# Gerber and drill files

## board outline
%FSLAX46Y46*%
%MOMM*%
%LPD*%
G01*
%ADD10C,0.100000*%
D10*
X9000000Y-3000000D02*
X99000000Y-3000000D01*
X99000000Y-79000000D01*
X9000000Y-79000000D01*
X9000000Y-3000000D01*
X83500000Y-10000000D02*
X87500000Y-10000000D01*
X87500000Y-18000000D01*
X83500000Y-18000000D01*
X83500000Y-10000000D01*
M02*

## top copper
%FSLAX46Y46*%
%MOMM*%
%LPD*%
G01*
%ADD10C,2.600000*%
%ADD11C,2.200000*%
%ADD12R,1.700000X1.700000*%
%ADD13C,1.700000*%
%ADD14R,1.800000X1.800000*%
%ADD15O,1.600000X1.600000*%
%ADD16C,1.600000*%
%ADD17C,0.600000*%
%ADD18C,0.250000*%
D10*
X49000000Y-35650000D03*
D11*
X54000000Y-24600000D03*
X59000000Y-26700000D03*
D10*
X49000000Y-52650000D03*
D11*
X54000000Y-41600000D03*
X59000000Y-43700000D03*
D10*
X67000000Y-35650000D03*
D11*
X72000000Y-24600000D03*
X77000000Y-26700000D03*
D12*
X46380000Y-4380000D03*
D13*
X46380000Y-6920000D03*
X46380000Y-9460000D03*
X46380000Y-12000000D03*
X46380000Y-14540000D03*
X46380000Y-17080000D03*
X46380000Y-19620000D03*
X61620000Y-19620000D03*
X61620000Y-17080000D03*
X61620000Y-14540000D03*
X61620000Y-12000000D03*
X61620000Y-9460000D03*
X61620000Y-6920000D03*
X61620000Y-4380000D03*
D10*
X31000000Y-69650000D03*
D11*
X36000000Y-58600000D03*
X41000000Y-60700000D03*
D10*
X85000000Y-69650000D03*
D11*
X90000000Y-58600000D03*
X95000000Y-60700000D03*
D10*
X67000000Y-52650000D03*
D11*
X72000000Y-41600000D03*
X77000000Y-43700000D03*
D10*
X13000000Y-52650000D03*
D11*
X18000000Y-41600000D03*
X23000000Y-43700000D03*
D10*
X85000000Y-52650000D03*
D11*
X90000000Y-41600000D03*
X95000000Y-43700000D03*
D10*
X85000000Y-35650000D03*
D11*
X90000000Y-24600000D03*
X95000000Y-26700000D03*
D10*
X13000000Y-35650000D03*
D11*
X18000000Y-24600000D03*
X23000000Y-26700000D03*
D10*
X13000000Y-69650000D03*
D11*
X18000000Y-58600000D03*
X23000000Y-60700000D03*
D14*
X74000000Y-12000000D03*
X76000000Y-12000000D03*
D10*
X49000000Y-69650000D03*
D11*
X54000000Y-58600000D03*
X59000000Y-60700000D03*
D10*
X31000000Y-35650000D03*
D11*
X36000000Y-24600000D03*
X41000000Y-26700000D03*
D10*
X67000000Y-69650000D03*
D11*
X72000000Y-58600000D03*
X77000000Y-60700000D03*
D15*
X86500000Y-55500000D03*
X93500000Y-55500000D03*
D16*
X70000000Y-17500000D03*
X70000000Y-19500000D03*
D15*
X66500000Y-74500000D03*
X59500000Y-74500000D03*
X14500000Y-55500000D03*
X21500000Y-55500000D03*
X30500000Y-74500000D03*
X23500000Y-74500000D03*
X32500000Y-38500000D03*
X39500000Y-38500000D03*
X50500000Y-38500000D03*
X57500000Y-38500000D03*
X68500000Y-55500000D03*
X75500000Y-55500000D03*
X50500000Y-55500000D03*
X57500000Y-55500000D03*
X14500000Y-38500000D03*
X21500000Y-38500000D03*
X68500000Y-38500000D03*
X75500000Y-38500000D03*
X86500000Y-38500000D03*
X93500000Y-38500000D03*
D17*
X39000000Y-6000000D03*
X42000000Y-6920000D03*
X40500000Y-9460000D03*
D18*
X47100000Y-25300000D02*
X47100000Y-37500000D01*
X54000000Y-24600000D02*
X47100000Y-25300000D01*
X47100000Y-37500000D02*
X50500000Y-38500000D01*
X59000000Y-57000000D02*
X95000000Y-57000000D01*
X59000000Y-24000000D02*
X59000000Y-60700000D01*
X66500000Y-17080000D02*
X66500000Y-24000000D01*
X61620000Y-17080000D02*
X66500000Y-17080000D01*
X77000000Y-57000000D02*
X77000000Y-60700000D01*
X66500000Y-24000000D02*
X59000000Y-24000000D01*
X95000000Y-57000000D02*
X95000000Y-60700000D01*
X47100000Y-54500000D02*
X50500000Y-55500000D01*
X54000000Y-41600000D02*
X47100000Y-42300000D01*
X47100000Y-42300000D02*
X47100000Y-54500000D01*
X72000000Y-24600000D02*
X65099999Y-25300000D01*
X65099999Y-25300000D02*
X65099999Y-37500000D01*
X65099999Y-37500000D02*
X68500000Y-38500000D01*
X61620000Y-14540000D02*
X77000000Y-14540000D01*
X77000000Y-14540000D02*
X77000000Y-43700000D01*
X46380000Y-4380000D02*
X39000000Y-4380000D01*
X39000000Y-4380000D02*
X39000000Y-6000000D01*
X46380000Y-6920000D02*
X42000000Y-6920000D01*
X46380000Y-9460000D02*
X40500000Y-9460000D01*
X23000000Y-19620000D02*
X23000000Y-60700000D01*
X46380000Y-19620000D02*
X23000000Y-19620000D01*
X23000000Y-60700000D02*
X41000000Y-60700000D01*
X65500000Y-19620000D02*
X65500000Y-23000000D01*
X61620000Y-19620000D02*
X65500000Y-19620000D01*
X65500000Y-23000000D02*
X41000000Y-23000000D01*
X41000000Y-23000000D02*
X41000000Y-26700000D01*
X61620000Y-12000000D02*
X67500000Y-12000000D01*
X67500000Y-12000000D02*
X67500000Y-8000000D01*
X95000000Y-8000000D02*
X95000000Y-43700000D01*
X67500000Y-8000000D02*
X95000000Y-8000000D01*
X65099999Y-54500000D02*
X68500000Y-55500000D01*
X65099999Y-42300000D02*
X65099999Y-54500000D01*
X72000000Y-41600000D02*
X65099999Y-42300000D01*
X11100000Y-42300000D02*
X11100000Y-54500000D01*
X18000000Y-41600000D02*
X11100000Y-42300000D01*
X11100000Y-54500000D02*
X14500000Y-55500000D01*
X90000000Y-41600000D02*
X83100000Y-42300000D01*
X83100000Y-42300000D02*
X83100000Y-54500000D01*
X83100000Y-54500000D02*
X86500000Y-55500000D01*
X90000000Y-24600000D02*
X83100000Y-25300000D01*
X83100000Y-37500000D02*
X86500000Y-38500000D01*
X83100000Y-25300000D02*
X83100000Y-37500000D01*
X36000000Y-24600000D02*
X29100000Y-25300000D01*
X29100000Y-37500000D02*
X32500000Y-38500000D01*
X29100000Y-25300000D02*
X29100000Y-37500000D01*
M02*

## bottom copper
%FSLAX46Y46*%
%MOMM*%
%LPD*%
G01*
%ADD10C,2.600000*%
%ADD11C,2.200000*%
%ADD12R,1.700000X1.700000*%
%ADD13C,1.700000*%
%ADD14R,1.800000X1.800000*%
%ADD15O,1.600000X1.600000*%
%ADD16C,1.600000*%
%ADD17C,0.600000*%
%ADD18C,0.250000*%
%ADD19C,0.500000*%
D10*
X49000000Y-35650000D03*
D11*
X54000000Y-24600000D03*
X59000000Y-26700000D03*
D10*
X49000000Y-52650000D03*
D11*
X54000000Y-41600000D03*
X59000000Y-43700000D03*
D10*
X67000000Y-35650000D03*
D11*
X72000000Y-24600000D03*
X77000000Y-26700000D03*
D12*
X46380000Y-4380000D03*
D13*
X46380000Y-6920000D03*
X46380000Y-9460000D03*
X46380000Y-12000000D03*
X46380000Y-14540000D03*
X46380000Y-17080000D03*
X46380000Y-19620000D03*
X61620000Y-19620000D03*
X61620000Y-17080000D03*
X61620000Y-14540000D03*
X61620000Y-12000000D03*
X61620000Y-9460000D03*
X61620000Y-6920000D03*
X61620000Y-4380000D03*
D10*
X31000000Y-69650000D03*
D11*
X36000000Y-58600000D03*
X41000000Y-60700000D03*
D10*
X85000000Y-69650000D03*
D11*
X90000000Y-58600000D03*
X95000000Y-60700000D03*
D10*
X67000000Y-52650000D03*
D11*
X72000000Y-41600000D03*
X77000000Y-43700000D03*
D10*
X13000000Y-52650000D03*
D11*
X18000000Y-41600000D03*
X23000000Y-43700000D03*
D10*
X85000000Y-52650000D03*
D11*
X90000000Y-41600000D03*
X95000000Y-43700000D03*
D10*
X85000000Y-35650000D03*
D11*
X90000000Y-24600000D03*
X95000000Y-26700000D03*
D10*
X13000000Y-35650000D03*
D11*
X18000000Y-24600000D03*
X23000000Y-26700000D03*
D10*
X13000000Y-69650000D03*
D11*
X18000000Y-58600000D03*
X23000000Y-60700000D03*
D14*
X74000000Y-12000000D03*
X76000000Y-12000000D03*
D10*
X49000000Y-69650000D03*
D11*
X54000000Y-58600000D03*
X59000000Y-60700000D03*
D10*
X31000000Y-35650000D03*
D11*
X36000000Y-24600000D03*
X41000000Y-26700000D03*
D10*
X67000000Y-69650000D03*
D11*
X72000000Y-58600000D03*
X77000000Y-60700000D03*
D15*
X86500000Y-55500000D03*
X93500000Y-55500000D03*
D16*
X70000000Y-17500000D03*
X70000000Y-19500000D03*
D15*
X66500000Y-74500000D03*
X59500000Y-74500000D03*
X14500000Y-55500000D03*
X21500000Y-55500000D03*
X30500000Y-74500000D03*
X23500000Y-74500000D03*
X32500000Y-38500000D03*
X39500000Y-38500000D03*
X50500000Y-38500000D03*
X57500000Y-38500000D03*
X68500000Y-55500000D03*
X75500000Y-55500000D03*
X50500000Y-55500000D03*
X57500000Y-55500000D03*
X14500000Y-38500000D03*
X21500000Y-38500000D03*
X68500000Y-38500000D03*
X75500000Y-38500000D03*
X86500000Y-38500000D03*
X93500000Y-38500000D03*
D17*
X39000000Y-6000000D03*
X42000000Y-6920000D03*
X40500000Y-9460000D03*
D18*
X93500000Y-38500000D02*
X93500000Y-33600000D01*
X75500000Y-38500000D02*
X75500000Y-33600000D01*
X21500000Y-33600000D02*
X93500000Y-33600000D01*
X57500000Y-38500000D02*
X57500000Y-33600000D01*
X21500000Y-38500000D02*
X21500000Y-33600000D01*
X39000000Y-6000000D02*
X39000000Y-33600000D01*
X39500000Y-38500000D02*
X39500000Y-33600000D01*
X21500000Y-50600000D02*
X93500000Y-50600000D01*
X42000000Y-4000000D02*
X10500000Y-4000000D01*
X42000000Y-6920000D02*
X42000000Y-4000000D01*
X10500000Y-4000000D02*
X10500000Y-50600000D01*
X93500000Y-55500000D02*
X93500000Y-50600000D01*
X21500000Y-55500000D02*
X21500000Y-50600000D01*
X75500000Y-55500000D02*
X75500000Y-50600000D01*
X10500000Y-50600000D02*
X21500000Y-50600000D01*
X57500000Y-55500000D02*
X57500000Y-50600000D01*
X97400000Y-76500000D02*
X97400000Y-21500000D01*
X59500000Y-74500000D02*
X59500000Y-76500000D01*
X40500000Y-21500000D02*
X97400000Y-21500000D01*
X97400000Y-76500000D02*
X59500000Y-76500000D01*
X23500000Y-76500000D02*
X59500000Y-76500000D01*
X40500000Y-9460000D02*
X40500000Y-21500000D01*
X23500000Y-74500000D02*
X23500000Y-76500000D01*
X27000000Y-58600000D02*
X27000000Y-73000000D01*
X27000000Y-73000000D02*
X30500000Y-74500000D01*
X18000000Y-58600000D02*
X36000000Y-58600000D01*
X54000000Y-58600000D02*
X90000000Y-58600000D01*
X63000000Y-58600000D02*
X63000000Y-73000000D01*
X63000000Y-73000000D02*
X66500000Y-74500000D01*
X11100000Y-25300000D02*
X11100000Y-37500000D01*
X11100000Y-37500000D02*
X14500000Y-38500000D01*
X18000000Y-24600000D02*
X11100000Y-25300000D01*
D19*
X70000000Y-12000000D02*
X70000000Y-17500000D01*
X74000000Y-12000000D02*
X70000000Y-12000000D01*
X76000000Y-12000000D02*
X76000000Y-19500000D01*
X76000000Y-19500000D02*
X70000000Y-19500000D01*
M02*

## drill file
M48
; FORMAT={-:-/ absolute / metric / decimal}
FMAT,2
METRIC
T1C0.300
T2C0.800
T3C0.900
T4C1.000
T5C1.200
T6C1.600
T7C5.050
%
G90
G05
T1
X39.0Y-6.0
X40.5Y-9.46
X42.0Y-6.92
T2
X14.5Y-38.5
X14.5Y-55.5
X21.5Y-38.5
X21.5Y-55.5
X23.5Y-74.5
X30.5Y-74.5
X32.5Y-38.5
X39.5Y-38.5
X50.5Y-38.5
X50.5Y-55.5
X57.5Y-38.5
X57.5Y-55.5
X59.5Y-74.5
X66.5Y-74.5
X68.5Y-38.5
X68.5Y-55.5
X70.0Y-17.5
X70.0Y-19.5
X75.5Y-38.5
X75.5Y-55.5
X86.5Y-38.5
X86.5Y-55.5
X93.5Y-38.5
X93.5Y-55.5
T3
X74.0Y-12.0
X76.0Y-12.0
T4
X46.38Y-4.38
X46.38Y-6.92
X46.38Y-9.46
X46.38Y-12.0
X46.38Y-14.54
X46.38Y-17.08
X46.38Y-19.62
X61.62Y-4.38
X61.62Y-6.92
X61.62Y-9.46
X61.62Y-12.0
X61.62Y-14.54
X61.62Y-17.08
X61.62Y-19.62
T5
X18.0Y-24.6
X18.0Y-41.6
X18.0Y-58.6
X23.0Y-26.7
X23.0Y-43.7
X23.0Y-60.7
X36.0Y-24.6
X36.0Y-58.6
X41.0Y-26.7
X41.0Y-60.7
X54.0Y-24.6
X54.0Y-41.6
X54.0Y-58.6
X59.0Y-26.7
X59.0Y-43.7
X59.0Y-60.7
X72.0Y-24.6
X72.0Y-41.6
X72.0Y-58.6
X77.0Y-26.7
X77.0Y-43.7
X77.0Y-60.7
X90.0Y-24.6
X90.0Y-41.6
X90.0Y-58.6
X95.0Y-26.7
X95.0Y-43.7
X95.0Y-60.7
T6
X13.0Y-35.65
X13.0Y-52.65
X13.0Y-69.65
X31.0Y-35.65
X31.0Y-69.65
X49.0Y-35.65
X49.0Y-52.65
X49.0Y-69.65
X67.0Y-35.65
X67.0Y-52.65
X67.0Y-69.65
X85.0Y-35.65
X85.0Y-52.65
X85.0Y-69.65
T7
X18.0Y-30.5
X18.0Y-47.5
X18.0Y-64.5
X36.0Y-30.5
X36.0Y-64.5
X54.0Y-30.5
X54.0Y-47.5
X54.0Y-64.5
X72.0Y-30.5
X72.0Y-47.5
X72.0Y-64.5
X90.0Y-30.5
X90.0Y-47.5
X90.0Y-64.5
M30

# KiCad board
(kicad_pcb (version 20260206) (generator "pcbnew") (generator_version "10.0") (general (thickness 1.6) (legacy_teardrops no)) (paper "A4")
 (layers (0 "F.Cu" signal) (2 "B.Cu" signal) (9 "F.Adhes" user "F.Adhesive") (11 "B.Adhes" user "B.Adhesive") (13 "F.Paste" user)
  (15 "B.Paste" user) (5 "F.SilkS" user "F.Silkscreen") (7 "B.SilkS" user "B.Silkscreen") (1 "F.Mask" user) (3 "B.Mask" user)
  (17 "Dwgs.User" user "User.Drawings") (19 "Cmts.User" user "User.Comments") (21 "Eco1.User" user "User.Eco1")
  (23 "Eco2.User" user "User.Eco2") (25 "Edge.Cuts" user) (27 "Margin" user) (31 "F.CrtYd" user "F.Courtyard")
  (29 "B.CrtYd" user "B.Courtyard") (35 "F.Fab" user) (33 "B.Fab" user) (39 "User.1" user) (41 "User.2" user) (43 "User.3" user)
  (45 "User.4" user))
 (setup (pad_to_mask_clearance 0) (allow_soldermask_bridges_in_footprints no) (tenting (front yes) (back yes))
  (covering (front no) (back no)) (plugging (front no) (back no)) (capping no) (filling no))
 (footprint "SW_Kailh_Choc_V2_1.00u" (layer "F.Cu") (at 54 30.5)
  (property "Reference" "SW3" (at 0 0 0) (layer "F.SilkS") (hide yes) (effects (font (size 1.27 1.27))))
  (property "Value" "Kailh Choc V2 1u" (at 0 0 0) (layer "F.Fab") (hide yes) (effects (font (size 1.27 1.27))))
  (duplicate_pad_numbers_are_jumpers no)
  (pad "" thru_hole circle (at -5 5.15) (size 2.6 2.6) (drill 1.6) (layers "*.Cu" "*.Mask") (remove_unused_layers no))
  (pad "" np_thru_hole circle (at 0 0) (size 5.05 5.05) (drill 5.05) (layers "*.Cu" "*.Mask"))
  (pad "1" thru_hole circle (at 0 -5.9) (size 2.2 2.2) (drill 1.2) (layers "*.Cu" "*.Mask") (remove_unused_layers no) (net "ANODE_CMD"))
  (pad "2" thru_hole circle (at 5 -3.8) (size 2.2 2.2) (drill 1.2) (layers "*.Cu" "*.Mask") (remove_unused_layers no) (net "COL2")))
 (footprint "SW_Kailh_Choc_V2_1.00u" (layer "F.Cu") (at 54 47.5)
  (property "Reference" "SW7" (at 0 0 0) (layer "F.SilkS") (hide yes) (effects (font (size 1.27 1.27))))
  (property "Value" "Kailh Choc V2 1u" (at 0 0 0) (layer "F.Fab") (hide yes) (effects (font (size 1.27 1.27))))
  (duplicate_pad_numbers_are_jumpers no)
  (pad "" thru_hole circle (at -5 5.15) (size 2.6 2.6) (drill 1.6) (layers "*.Cu" "*.Mask") (remove_unused_layers no))
  (pad "" np_thru_hole circle (at 0 0) (size 5.05 5.05) (drill 5.05) (layers "*.Cu" "*.Mask"))
  (pad "1" thru_hole circle (at 0 -5.9) (size 2.2 2.2) (drill 1.2) (layers "*.Cu" "*.Mask") (remove_unused_layers no) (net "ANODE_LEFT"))
  (pad "2" thru_hole circle (at 5 -3.8) (size 2.2 2.2) (drill 1.2) (layers "*.Cu" "*.Mask") (remove_unused_layers no) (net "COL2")))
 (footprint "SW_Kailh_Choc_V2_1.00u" (layer "F.Cu") (at 72 30.5)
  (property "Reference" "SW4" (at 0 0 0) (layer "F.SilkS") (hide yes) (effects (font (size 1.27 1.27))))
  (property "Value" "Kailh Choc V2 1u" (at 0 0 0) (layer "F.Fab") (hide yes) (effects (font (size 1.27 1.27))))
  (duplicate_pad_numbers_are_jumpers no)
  (pad "" thru_hole circle (at -5 5.15) (size 2.6 2.6) (drill 1.6) (layers "*.Cu" "*.Mask") (remove_unused_layers no))
  (pad "" np_thru_hole circle (at 0 0) (size 5.05 5.05) (drill 5.05) (layers "*.Cu" "*.Mask"))
  (pad "1" thru_hole circle (at 0 -5.9) (size 2.2 2.2) (drill 1.2) (layers "*.Cu" "*.Mask") (remove_unused_layers no) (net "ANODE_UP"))
  (pad "2" thru_hole circle (at 5 -3.8) (size 2.2 2.2) (drill 1.2) (layers "*.Cu" "*.Mask") (remove_unused_layers no) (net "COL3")))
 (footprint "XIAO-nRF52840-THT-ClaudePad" (layer "F.Cu") (at 54 12)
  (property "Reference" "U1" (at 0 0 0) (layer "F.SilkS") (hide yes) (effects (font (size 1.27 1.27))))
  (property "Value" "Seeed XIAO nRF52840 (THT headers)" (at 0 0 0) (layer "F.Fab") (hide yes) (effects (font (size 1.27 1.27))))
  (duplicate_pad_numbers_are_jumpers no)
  (pad "1" thru_hole rect (at -7.62 -7.62) (size 1.7 1.7) (drill 1) (layers "*.Cu" "*.Mask") (remove_unused_layers no) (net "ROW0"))
  (pad "2" thru_hole circle (at -7.62 -5.08) (size 1.7 1.7) (drill 1) (layers "*.Cu" "*.Mask") (remove_unused_layers no) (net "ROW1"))
  (pad "3" thru_hole circle (at -7.62 -2.54) (size 1.7 1.7) (drill 1) (layers "*.Cu" "*.Mask") (remove_unused_layers no) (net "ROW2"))
  (pad "4" thru_hole circle (at -7.62 0) (size 1.7 1.7) (drill 1) (layers "*.Cu" "*.Mask") (remove_unused_layers no))
  (pad "5" thru_hole circle (at -7.62 2.54) (size 1.7 1.7) (drill 1) (layers "*.Cu" "*.Mask") (remove_unused_layers no))
  (pad "6" thru_hole circle (at -7.62 5.08) (size 1.7 1.7) (drill 1) (layers "*.Cu" "*.Mask") (remove_unused_layers no))
  (pad "7" thru_hole circle (at -7.62 7.62) (size 1.7 1.7) (drill 1) (layers "*.Cu" "*.Mask") (remove_unused_layers no) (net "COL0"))
  (pad "8" thru_hole circle (at 7.62 7.62) (size 1.7 1.7) (drill 1) (layers "*.Cu" "*.Mask") (remove_unused_layers no) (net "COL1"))
  (pad "9" thru_hole circle (at 7.62 5.08) (size 1.7 1.7) (drill 1) (layers "*.Cu" "*.Mask") (remove_unused_layers no) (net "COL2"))
  (pad "10" thru_hole circle (at 7.62 2.54) (size 1.7 1.7) (drill 1) (layers "*.Cu" "*.Mask") (remove_unused_layers no) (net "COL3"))
  (pad "11" thru_hole circle (at 7.62 0) (size 1.7 1.7) (drill 1) (layers "*.Cu" "*.Mask") (remove_unused_layers no) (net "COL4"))
  (pad "12" thru_hole circle (at 7.62 -2.54) (size 1.7 1.7) (drill 1) (layers "*.Cu" "*.Mask") (remove_unused_layers no))
  (pad "13" thru_hole circle (at 7.62 -5.08) (size 1.7 1.7) (drill 1) (layers "*.Cu" "*.Mask") (remove_unused_layers no))
  (pad "14" thru_hole circle (at 7.62 -7.62) (size 1.7 1.7) (drill 1) (layers "*.Cu" "*.Mask") (remove_unused_layers no)))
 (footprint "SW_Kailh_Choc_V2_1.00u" (layer "F.Cu") (at 36 64.5)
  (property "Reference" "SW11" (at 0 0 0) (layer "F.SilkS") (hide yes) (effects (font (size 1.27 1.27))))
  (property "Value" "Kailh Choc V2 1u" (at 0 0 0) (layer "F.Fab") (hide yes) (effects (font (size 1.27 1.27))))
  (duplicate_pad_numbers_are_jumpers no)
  (pad "" thru_hole circle (at -5 5.15) (size 2.6 2.6) (drill 1.6) (layers "*.Cu" "*.Mask") (remove_unused_layers no))
  (pad "" np_thru_hole circle (at 0 0) (size 5.05 5.05) (drill 5.05) (layers "*.Cu" "*.Mask"))
  (pad "1" thru_hole circle (at 0 -5.9) (size 2.2 2.2) (drill 1.2) (layers "*.Cu" "*.Mask") (remove_unused_layers no) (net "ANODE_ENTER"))
  (pad "2" thru_hole circle (at 5 -3.8) (size 2.2 2.2) (drill 1.2) (layers "*.Cu" "*.Mask") (remove_unused_layers no) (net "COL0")))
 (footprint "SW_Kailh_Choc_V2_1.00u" (layer "F.Cu") (at 90 64.5)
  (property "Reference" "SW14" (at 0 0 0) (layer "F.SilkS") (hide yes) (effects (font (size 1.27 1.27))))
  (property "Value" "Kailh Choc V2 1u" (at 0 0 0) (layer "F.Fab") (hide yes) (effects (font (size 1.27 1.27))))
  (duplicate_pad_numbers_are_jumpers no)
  (pad "" thru_hole circle (at -5 5.15) (size 2.6 2.6) (drill 1.6) (layers "*.Cu" "*.Mask") (remove_unused_layers no))
  (pad "" np_thru_hole circle (at 0 0) (size 5.05 5.05) (drill 5.05) (layers "*.Cu" "*.Mask"))
  (pad "1" thru_hole circle (at 0 -5.9) (size 2.2 2.2) (drill 1.2) (layers "*.Cu" "*.Mask") (remove_unused_layers no) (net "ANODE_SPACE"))
  (pad "2" thru_hole circle (at 5 -3.8) (size 2.2 2.2) (drill 1.2) (layers "*.Cu" "*.Mask") (remove_unused_layers no) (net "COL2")))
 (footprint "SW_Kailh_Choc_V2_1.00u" (layer "F.Cu") (at 72 47.5)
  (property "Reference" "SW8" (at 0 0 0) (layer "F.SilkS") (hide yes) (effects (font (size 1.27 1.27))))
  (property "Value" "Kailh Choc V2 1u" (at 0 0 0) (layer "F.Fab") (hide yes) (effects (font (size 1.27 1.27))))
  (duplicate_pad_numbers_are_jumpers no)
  (pad "" thru_hole circle (at -5 5.15) (size 2.6 2.6) (drill 1.6) (layers "*.Cu" "*.Mask") (remove_unused_layers no))
  (pad "" np_thru_hole circle (at 0 0) (size 5.05 5.05) (drill 5.05) (layers "*.Cu" "*.Mask"))
  (pad "1" thru_hole circle (at 0 -5.9) (size 2.2 2.2) (drill 1.2) (layers "*.Cu" "*.Mask") (remove_unused_layers no) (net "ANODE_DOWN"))
  (pad "2" thru_hole circle (at 5 -3.8) (size 2.2 2.2) (drill 1.2) (layers "*.Cu" "*.Mask") (remove_unused_layers no) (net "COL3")))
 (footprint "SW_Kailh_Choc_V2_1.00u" (layer "F.Cu") (at 18 47.5)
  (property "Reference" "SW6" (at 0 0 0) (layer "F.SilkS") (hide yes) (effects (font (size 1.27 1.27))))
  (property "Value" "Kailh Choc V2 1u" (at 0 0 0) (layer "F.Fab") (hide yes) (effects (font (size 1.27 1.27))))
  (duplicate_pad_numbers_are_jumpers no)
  (pad "" thru_hole circle (at -5 5.15) (size 2.6 2.6) (drill 1.6) (layers "*.Cu" "*.Mask") (remove_unused_layers no))
  (pad "" np_thru_hole circle (at 0 0) (size 5.05 5.05) (drill 5.05) (layers "*.Cu" "*.Mask"))
  (pad "1" thru_hole circle (at 0 -5.9) (size 2.2 2.2) (drill 1.2) (layers "*.Cu" "*.Mask") (remove_unused_layers no) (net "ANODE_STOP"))
  (pad "2" thru_hole circle (at 5 -3.8) (size 2.2 2.2) (drill 1.2) (layers "*.Cu" "*.Mask") (remove_unused_layers no) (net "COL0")))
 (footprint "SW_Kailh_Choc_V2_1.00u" (layer "F.Cu") (at 90 47.5)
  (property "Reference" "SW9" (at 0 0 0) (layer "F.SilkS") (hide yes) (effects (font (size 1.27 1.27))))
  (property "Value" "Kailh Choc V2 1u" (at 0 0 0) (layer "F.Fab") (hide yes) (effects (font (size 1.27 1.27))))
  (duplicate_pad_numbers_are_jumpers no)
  (pad "" thru_hole circle (at -5 5.15) (size 2.6 2.6) (drill 1.6) (layers "*.Cu" "*.Mask") (remove_unused_layers no))
  (pad "" np_thru_hole circle (at 0 0) (size 5.05 5.05) (drill 5.05) (layers "*.Cu" "*.Mask"))
  (pad "1" thru_hole circle (at 0 -5.9) (size 2.2 2.2) (drill 1.2) (layers "*.Cu" "*.Mask") (remove_unused_layers no) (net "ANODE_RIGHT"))
  (pad "2" thru_hole circle (at 5 -3.8) (size 2.2 2.2) (drill 1.2) (layers "*.Cu" "*.Mask") (remove_unused_layers no) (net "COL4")))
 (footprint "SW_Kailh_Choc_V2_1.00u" (layer "F.Cu") (at 90 30.5)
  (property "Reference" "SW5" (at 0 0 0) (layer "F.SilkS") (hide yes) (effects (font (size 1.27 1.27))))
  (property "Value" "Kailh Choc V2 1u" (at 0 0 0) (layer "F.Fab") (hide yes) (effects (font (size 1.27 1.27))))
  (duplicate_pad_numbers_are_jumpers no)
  (pad "" thru_hole circle (at -5 5.15) (size 2.6 2.6) (drill 1.6) (layers "*.Cu" "*.Mask") (remove_unused_layers no))
  (pad "" np_thru_hole circle (at 0 0) (size 5.05 5.05) (drill 5.05) (layers "*.Cu" "*.Mask"))
  (pad "1" thru_hole circle (at 0 -5.9) (size 2.2 2.2) (drill 1.2) (layers "*.Cu" "*.Mask") (remove_unused_layers no) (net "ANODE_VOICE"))
  (pad "2" thru_hole circle (at 5 -3.8) (size 2.2 2.2) (drill 1.2) (layers "*.Cu" "*.Mask") (remove_unused_layers no) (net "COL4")))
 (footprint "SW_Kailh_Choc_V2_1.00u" (layer "F.Cu") (at 18 30.5)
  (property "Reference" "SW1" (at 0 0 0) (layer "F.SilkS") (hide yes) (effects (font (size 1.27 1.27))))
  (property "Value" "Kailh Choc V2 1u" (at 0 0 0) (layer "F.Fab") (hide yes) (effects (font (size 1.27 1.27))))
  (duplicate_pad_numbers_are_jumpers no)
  (pad "" thru_hole circle (at -5 5.15) (size 2.6 2.6) (drill 1.6) (layers "*.Cu" "*.Mask") (remove_unused_layers no))
  (pad "" np_thru_hole circle (at 0 0) (size 5.05 5.05) (drill 5.05) (layers "*.Cu" "*.Mask"))
  (pad "1" thru_hole circle (at 0 -5.9) (size 2.2 2.2) (drill 1.2) (layers "*.Cu" "*.Mask") (remove_unused_layers no) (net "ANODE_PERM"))
  (pad "2" thru_hole circle (at 5 -3.8) (size 2.2 2.2) (drill 1.2) (layers "*.Cu" "*.Mask") (remove_unused_layers no) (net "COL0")))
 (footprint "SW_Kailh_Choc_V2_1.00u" (layer "F.Cu") (at 18 64.5)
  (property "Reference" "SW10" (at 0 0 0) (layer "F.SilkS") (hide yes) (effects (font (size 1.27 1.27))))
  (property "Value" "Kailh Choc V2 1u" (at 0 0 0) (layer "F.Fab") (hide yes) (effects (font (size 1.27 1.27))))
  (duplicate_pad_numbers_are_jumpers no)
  (pad "" thru_hole circle (at -5 5.15) (size 2.6 2.6) (drill 1.6) (layers "*.Cu" "*.Mask") (remove_unused_layers no))
  (pad "" np_thru_hole circle (at 0 0) (size 5.05 5.05) (drill 5.05) (layers "*.Cu" "*.Mask"))
  (pad "1" thru_hole circle (at 0 -5.9) (size 2.2 2.2) (drill 1.2) (layers "*.Cu" "*.Mask") (remove_unused_layers no) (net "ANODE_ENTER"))
  (pad "2" thru_hole circle (at 5 -3.8) (size 2.2 2.2) (drill 1.2) (layers "*.Cu" "*.Mask") (remove_unused_layers no) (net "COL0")))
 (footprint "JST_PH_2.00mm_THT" (layer "F.Cu") (at 74 12)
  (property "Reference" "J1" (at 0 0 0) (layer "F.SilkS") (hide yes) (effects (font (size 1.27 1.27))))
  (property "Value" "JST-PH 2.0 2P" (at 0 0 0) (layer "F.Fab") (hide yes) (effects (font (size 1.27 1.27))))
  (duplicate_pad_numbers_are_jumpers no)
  (pad "1" thru_hole rect (at 0 0) (size 1.8 1.8) (drill 0.9) (layers "*.Cu" "*.Mask") (remove_unused_layers no) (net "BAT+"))
  (pad "2" thru_hole rect (at 2 0) (size 1.8 1.8) (drill 0.9) (layers "*.Cu" "*.Mask") (remove_unused_layers no) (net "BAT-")))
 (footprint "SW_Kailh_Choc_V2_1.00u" (layer "F.Cu") (at 54 64.5)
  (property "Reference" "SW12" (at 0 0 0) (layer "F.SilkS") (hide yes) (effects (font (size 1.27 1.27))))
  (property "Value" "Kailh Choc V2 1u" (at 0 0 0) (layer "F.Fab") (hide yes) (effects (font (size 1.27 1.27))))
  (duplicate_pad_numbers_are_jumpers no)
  (pad "" thru_hole circle (at -5 5.15) (size 2.6 2.6) (drill 1.6) (layers "*.Cu" "*.Mask") (remove_unused_layers no))
  (pad "" np_thru_hole circle (at 0 0) (size 5.05 5.05) (drill 5.05) (layers "*.Cu" "*.Mask"))
  (pad "1" thru_hole circle (at 0 -5.9) (size 2.2 2.2) (drill 1.2) (layers "*.Cu" "*.Mask") (remove_unused_layers no) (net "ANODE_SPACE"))
  (pad "2" thru_hole circle (at 5 -3.8) (size 2.2 2.2) (drill 1.2) (layers "*.Cu" "*.Mask") (remove_unused_layers no) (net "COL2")))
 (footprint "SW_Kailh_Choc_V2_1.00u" (layer "F.Cu") (at 36 30.5)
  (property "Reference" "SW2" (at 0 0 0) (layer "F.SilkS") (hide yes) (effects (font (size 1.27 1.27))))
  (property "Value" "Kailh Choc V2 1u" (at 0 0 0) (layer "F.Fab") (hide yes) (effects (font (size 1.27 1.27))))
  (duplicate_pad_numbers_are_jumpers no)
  (pad "" thru_hole circle (at -5 5.15) (size 2.6 2.6) (drill 1.6) (layers "*.Cu" "*.Mask") (remove_unused_layers no))
  (pad "" np_thru_hole circle (at 0 0) (size 5.05 5.05) (drill 5.05) (layers "*.Cu" "*.Mask"))
  (pad "1" thru_hole circle (at 0 -5.9) (size 2.2 2.2) (drill 1.2) (layers "*.Cu" "*.Mask") (remove_unused_layers no) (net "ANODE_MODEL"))
  (pad "2" thru_hole circle (at 5 -3.8) (size 2.2 2.2) (drill 1.2) (layers "*.Cu" "*.Mask") (remove_unused_layers no) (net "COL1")))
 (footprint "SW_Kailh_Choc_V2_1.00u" (layer "F.Cu") (at 72 64.5)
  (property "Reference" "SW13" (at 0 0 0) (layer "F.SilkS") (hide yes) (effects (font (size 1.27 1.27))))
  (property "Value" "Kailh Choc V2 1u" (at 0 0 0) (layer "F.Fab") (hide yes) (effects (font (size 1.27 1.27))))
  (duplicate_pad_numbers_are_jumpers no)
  (pad "" thru_hole circle (at -5 5.15) (size 2.6 2.6) (drill 1.6) (layers "*.Cu" "*.Mask") (remove_unused_layers no))
  (pad "" np_thru_hole circle (at 0 0) (size 5.05 5.05) (drill 5.05) (layers "*.Cu" "*.Mask"))
  (pad "1" thru_hole circle (at 0 -5.9) (size 2.2 2.2) (drill 1.2) (layers "*.Cu" "*.Mask") (remove_unused_layers no) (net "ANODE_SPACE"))
  (pad "2" thru_hole circle (at 5 -3.8) (size 2.2 2.2) (drill 1.2) (layers "*.Cu" "*.Mask") (remove_unused_layers no) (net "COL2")))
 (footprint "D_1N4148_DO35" (layer "B.Cu") (at 90 55.5)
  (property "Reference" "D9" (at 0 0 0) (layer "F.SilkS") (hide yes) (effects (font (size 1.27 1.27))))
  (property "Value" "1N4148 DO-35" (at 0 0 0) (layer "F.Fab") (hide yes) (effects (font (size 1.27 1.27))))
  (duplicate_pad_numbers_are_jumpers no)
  (pad "1" thru_hole oval (at -3.5 0) (size 1.6 1.6) (drill 0.8) (layers "*.Cu" "*.Mask") (remove_unused_layers no) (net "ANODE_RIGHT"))
  (pad "2" thru_hole oval (at 3.5 0) (size 1.6 1.6) (drill 0.8) (layers "*.Cu" "*.Mask") (remove_unused_layers no) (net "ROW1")))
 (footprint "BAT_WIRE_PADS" (layer "B.Cu") (at 70 17.5)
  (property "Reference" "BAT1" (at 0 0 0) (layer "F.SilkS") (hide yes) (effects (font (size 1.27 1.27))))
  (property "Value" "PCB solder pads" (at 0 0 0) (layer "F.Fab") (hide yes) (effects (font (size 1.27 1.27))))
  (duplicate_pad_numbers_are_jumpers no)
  (pad "1" thru_hole circle (at 0 0) (size 1.6 1.6) (drill 0.8) (layers "*.Cu" "*.Mask") (remove_unused_layers no) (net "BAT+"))
  (pad "2" thru_hole circle (at 0 2) (size 1.6 1.6) (drill 0.8) (layers "*.Cu" "*.Mask") (remove_unused_layers no) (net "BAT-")))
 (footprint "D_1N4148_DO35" (layer "B.Cu") (at 63 74.5 180)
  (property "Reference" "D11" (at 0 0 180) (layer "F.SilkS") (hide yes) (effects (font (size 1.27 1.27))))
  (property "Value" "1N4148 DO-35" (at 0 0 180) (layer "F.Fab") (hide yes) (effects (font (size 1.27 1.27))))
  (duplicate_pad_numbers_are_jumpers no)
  (pad "1" thru_hole oval (at -3.5 0 180) (size 1.6 1.6) (drill 0.8) (layers "*.Cu" "*.Mask") (remove_unused_layers no) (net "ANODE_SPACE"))
  (pad "2" thru_hole oval (at 3.5 0 180) (size 1.6 1.6) (drill 0.8) (layers "*.Cu" "*.Mask") (remove_unused_layers no) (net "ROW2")))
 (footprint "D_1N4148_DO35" (layer "B.Cu") (at 18 55.5)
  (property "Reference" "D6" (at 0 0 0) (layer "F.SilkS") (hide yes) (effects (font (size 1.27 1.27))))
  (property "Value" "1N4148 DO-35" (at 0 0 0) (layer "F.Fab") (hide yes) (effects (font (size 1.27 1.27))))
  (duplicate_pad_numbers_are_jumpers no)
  (pad "1" thru_hole oval (at -3.5 0) (size 1.6 1.6) (drill 0.8) (layers "*.Cu" "*.Mask") (remove_unused_layers no) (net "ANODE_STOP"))
  (pad "2" thru_hole oval (at 3.5 0) (size 1.6 1.6) (drill 0.8) (layers "*.Cu" "*.Mask") (remove_unused_layers no) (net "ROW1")))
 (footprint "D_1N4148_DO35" (layer "B.Cu") (at 27 74.5 180)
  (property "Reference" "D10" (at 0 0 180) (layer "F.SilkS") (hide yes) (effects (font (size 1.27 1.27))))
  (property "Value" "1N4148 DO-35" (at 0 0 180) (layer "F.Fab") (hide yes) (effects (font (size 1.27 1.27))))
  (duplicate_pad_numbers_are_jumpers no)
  (pad "1" thru_hole oval (at -3.5 0 180) (size 1.6 1.6) (drill 0.8) (layers "*.Cu" "*.Mask") (remove_unused_layers no) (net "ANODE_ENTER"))
  (pad "2" thru_hole oval (at 3.5 0 180) (size 1.6 1.6) (drill 0.8) (layers "*.Cu" "*.Mask") (remove_unused_layers no) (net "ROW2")))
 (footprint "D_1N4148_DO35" (layer "B.Cu") (at 36 38.5)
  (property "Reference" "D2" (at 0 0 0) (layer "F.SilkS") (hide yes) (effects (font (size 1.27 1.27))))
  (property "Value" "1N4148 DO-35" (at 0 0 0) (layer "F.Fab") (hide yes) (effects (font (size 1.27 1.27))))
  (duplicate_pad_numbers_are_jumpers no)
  (pad "1" thru_hole oval (at -3.5 0) (size 1.6 1.6) (drill 0.8) (layers "*.Cu" "*.Mask") (remove_unused_layers no) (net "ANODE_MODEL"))
  (pad "2" thru_hole oval (at 3.5 0) (size 1.6 1.6) (drill 0.8) (layers "*.Cu" "*.Mask") (remove_unused_layers no) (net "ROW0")))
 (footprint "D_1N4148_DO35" (layer "B.Cu") (at 54 38.5)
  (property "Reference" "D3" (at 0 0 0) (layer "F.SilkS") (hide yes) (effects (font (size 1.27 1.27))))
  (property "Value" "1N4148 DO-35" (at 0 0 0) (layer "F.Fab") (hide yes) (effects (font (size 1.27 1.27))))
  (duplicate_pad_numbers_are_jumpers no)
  (pad "1" thru_hole oval (at -3.5 0) (size 1.6 1.6) (drill 0.8) (layers "*.Cu" "*.Mask") (remove_unused_layers no) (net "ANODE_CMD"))
  (pad "2" thru_hole oval (at 3.5 0) (size 1.6 1.6) (drill 0.8) (layers "*.Cu" "*.Mask") (remove_unused_layers no) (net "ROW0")))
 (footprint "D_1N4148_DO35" (layer "B.Cu") (at 72 55.5)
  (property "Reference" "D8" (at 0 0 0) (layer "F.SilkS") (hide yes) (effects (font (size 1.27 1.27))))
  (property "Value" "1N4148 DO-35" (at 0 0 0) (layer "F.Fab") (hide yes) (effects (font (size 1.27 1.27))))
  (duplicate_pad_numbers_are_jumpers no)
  (pad "1" thru_hole oval (at -3.5 0) (size 1.6 1.6) (drill 0.8) (layers "*.Cu" "*.Mask") (remove_unused_layers no) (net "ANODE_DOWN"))
  (pad "2" thru_hole oval (at 3.5 0) (size 1.6 1.6) (drill 0.8) (layers "*.Cu" "*.Mask") (remove_unused_layers no) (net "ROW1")))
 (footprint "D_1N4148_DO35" (layer "B.Cu") (at 54 55.5)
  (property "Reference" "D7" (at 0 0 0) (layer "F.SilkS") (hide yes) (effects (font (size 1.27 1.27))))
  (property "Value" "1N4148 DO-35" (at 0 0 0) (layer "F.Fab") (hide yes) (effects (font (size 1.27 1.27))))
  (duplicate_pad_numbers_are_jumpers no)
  (pad "1" thru_hole oval (at -3.5 0) (size 1.6 1.6) (drill 0.8) (layers "*.Cu" "*.Mask") (remove_unused_layers no) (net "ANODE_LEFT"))
  (pad "2" thru_hole oval (at 3.5 0) (size 1.6 1.6) (drill 0.8) (layers "*.Cu" "*.Mask") (remove_unused_layers no) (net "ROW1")))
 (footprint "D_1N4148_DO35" (layer "B.Cu") (at 18 38.5)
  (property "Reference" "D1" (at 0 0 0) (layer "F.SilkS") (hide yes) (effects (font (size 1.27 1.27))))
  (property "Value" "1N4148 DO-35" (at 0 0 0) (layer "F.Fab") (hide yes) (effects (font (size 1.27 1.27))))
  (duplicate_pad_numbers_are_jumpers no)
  (pad "1" thru_hole oval (at -3.5 0) (size 1.6 1.6) (drill 0.8) (layers "*.Cu" "*.Mask") (remove_unused_layers no) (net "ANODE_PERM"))
  (pad "2" thru_hole oval (at 3.5 0) (size 1.6 1.6) (drill 0.8) (layers "*.Cu" "*.Mask") (remove_unused_layers no) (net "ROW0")))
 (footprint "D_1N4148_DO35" (layer "B.Cu") (at 72 38.5)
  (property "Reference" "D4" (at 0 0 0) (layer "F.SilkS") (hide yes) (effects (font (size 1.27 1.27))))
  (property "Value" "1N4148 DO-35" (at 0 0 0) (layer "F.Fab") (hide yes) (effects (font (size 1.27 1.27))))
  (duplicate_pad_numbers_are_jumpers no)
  (pad "1" thru_hole oval (at -3.5 0) (size 1.6 1.6) (drill 0.8) (layers "*.Cu" "*.Mask") (remove_unused_layers no) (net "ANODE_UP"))
  (pad "2" thru_hole oval (at 3.5 0) (size 1.6 1.6) (drill 0.8) (layers "*.Cu" "*.Mask") (remove_unused_layers no) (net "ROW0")))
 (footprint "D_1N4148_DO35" (layer "B.Cu") (at 90 38.5)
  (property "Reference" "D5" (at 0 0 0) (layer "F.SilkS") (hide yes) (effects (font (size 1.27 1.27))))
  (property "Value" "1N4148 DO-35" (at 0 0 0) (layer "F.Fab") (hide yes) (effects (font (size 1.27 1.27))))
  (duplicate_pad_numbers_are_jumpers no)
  (pad "1" thru_hole oval (at -3.5 0) (size 1.6 1.6) (drill 0.8) (layers "*.Cu" "*.Mask") (remove_unused_layers no) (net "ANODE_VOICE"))
  (pad "2" thru_hole oval (at 3.5 0) (size 1.6 1.6) (drill 0.8) (layers "*.Cu" "*.Mask") (remove_unused_layers no) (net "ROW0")))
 (gr_rect (start 9 3) (end 99 79) (stroke (width 0.1) (type default)) (fill no) (layer "Edge.Cuts"))
 (gr_rect (start 83.5 10) (end 87.5 18) (stroke (width 0.1) (type default)) (fill no) (layer "Edge.Cuts"))
 (segment (start 47.1 25.3) (end 47.1 37.5) (width 0.25) (layer "F.Cu") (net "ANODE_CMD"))
 (segment (start 54 24.6) (end 47.1 25.3) (width 0.25) (layer "F.Cu") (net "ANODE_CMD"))
 (segment (start 47.1 37.5) (end 50.5 38.5) (width 0.25) (layer "F.Cu") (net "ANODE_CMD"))
 (segment (start 59 57) (end 95 57) (width 0.25) (layer "F.Cu") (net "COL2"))
 (segment (start 59 24) (end 59 60.7) (width 0.25) (layer "F.Cu") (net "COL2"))
 (segment (start 66.5 17.08) (end 66.5 24) (width 0.25) (layer "F.Cu") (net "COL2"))
 (segment (start 61.62 17.08) (end 66.5 17.08) (width 0.25) (layer "F.Cu") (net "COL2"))
 (segment (start 77 57) (end 77 60.7) (width 0.25) (layer "F.Cu") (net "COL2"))
 (segment (start 66.5 24) (end 59 24) (width 0.25) (layer "F.Cu") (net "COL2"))
 (segment (start 95 57) (end 95 60.7) (width 0.25) (layer "F.Cu") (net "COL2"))
 (segment (start 47.1 54.5) (end 50.5 55.5) (width 0.25) (layer "F.Cu") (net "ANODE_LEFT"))
 (segment (start 54 41.6) (end 47.1 42.3) (width 0.25) (layer "F.Cu") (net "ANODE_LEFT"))
 (segment (start 47.1 42.3) (end 47.1 54.5) (width 0.25) (layer "F.Cu") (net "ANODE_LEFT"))
 (segment (start 72 24.6) (end 65.099999 25.3) (width 0.25) (layer "F.Cu") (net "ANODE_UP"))
 (segment (start 65.099999 25.3) (end 65.099999 37.5) (width 0.25) (layer "F.Cu") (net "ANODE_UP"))
 (segment (start 65.099999 37.5) (end 68.5 38.5) (width 0.25) (layer "F.Cu") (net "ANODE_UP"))
 (segment (start 61.62 14.54) (end 77 14.54) (width 0.25) (layer "F.Cu") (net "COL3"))
 (segment (start 77 14.54) (end 77 43.7) (width 0.25) (layer "F.Cu") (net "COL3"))
 (segment (start 46.38 4.38) (end 39 4.38) (width 0.25) (layer "F.Cu") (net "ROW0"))
 (segment (start 39 4.38) (end 39 6) (width 0.25) (layer "F.Cu") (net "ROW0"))
 (via (at 39 6) (size 0.6) (drill 0.3) (layers "F.Cu" "B.Cu") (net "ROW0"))
 (segment (start 93.5 38.5) (end 93.5 33.6) (width 0.25) (layer "B.Cu") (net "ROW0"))
 (segment (start 75.5 38.5) (end 75.5 33.6) (width 0.25) (layer "B.Cu") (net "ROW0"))
 (segment (start 21.5 33.6) (end 93.5 33.6) (width 0.25) (layer "B.Cu") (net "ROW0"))
 (segment (start 57.5 38.5) (end 57.5 33.6) (width 0.25) (layer "B.Cu") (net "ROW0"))
 (segment (start 21.5 38.5) (end 21.5 33.6) (width 0.25) (layer "B.Cu") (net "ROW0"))
 (segment (start 39 6) (end 39 33.6) (width 0.25) (layer "B.Cu") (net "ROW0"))
 (segment (start 39.5 38.5) (end 39.5 33.6) (width 0.25) (layer "B.Cu") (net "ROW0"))
 (segment (start 46.38 6.92) (end 42 6.92) (width 0.25) (layer "F.Cu") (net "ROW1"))
 (via (at 42 6.92) (size 0.6) (drill 0.3) (layers "F.Cu" "B.Cu") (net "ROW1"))
 (segment (start 21.5 50.6) (end 93.5 50.6) (width 0.25) (layer "B.Cu") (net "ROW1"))
 (segment (start 42 4) (end 10.5 4) (width 0.25) (layer "B.Cu") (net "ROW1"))
 (segment (start 42 6.92) (end 42 4) (width 0.25) (layer "B.Cu") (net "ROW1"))
 (segment (start 10.5 4) (end 10.5 50.6) (width 0.25) (layer "B.Cu") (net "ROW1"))
 (segment (start 93.5 55.5) (end 93.5 50.6) (width 0.25) (layer "B.Cu") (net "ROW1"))
 (segment (start 21.5 55.5) (end 21.5 50.6) (width 0.25) (layer "B.Cu") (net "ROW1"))
 (segment (start 75.5 55.5) (end 75.5 50.6) (width 0.25) (layer "B.Cu") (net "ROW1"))
 (segment (start 10.5 50.6) (end 21.5 50.6) (width 0.25) (layer "B.Cu") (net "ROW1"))
 (segment (start 57.5 55.5) (end 57.5 50.6) (width 0.25) (layer "B.Cu") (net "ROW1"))
 (segment (start 46.38 9.46) (end 40.5 9.46) (width 0.25) (layer "F.Cu") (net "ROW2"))
 (via (at 40.5 9.46) (size 0.6) (drill 0.3) (layers "F.Cu" "B.Cu") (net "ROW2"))
 (segment (start 97.4 76.5) (end 97.4 21.5) (width 0.25) (layer "B.Cu") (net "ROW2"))
 (segment (start 59.5 74.5) (end 59.5 76.5) (width 0.25) (layer "B.Cu") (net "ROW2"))
 (segment (start 40.5 21.5) (end 97.4 21.5) (width 0.25) (layer "B.Cu") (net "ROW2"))
 (segment (start 97.4 76.5) (end 59.5 76.5) (width 0.25) (layer "B.Cu") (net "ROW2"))
 (segment (start 23.5 76.5) (end 59.5 76.5) (width 0.25) (layer "B.Cu") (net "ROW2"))
 (segment (start 40.5 9.46) (end 40.5 21.5) (width 0.25) (layer "B.Cu") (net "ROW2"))
 (segment (start 23.5 74.5) (end 23.5 76.5) (width 0.25) (layer "B.Cu") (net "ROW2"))
 (segment (start 23 19.62) (end 23 60.7) (width 0.25) (layer "F.Cu") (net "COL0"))
 (segment (start 46.38 19.62) (end 23 19.62) (width 0.25) (layer "F.Cu") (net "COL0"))
 (segment (start 23 60.7) (end 41 60.7) (width 0.25) (layer "F.Cu") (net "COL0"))
 (segment (start 65.5 19.62) (end 65.5 23) (width 0.25) (layer "F.Cu") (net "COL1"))
 (segment (start 61.62 19.62) (end 65.5 19.62) (width 0.25) (layer "F.Cu") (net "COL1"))
 (segment (start 65.5 23) (end 41 23) (width 0.25) (layer "F.Cu") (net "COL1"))
 (segment (start 41 23) (end 41 26.7) (width 0.25) (layer "F.Cu") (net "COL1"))
 (segment (start 61.62 12) (end 67.5 12) (width 0.25) (layer "F.Cu") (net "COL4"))
 (segment (start 67.5 12) (end 67.5 8) (width 0.25) (layer "F.Cu") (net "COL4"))
 (segment (start 95 8) (end 95 43.7) (width 0.25) (layer "F.Cu") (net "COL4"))
 (segment (start 67.5 8) (end 95 8) (width 0.25) (layer "F.Cu") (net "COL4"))
 (segment (start 27 58.6) (end 27 73) (width 0.25) (layer "B.Cu") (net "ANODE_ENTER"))
 (segment (start 27 73) (end 30.5 74.5) (width 0.25) (layer "B.Cu") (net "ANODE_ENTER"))
 (segment (start 18 58.6) (end 36 58.6) (width 0.25) (layer "B.Cu") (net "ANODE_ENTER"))
 (segment (start 54 58.6) (end 90 58.6) (width 0.25) (layer "B.Cu") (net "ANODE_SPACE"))
 (segment (start 63 58.6) (end 63 73) (width 0.25) (layer "B.Cu") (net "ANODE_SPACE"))
 (segment (start 63 73) (end 66.5 74.5) (width 0.25) (layer "B.Cu") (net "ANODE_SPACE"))
 (segment (start 65.099999 54.5) (end 68.5 55.5) (width 0.25) (layer "F.Cu") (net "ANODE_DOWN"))
 (segment (start 65.099999 42.3) (end 65.099999 54.5) (width 0.25) (layer "F.Cu") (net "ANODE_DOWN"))
 (segment (start 72 41.6) (end 65.099999 42.3) (width 0.25) (layer "F.Cu") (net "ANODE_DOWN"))
 (segment (start 11.1 42.3) (end 11.1 54.5) (width 0.25) (layer "F.Cu") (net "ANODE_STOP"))
 (segment (start 18 41.6) (end 11.1 42.3) (width 0.25) (layer "F.Cu") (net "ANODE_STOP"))
 (segment (start 11.1 54.5) (end 14.5 55.5) (width 0.25) (layer "F.Cu") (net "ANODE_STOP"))
 (segment (start 90 41.6) (end 83.1 42.3) (width 0.25) (layer "F.Cu") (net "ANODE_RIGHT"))
 (segment (start 83.1 42.3) (end 83.1 54.5) (width 0.25) (layer "F.Cu") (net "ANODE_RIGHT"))
 (segment (start 83.1 54.5) (end 86.5 55.5) (width 0.25) (layer "F.Cu") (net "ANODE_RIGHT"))
 (segment (start 90 24.6) (end 83.1 25.3) (width 0.25) (layer "F.Cu") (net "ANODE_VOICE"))
 (segment (start 83.1 37.5) (end 86.5 38.5) (width 0.25) (layer "F.Cu") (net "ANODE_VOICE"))
 (segment (start 83.1 25.3) (end 83.1 37.5) (width 0.25) (layer "F.Cu") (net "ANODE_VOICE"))
 (segment (start 11.1 25.3) (end 11.1 37.5) (width 0.25) (layer "B.Cu") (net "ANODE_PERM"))
 (segment (start 11.1 37.5) (end 14.5 38.5) (width 0.25) (layer "B.Cu") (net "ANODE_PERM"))
 (segment (start 18 24.6) (end 11.1 25.3) (width 0.25) (layer "B.Cu") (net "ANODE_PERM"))
 (segment (start 70 12) (end 70 17.5) (width 0.5) (layer "B.Cu") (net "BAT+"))
 (segment (start 74 12) (end 70 12) (width 0.5) (layer "B.Cu") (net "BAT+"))
 (segment (start 76 12) (end 76 19.5) (width 0.5) (layer "B.Cu") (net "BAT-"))
 (segment (start 76 19.5) (end 70 19.5) (width 0.5) (layer "B.Cu") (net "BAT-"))
 (segment (start 36 24.6) (end 29.1 25.3) (width 0.25) (layer "F.Cu") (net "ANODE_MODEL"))
 (segment (start 29.1 37.5) (end 32.5 38.5) (width 0.25) (layer "F.Cu") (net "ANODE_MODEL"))
 (segment (start 29.1 25.3) (end 29.1 37.5) (width 0.25) (layer "F.Cu") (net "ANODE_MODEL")))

